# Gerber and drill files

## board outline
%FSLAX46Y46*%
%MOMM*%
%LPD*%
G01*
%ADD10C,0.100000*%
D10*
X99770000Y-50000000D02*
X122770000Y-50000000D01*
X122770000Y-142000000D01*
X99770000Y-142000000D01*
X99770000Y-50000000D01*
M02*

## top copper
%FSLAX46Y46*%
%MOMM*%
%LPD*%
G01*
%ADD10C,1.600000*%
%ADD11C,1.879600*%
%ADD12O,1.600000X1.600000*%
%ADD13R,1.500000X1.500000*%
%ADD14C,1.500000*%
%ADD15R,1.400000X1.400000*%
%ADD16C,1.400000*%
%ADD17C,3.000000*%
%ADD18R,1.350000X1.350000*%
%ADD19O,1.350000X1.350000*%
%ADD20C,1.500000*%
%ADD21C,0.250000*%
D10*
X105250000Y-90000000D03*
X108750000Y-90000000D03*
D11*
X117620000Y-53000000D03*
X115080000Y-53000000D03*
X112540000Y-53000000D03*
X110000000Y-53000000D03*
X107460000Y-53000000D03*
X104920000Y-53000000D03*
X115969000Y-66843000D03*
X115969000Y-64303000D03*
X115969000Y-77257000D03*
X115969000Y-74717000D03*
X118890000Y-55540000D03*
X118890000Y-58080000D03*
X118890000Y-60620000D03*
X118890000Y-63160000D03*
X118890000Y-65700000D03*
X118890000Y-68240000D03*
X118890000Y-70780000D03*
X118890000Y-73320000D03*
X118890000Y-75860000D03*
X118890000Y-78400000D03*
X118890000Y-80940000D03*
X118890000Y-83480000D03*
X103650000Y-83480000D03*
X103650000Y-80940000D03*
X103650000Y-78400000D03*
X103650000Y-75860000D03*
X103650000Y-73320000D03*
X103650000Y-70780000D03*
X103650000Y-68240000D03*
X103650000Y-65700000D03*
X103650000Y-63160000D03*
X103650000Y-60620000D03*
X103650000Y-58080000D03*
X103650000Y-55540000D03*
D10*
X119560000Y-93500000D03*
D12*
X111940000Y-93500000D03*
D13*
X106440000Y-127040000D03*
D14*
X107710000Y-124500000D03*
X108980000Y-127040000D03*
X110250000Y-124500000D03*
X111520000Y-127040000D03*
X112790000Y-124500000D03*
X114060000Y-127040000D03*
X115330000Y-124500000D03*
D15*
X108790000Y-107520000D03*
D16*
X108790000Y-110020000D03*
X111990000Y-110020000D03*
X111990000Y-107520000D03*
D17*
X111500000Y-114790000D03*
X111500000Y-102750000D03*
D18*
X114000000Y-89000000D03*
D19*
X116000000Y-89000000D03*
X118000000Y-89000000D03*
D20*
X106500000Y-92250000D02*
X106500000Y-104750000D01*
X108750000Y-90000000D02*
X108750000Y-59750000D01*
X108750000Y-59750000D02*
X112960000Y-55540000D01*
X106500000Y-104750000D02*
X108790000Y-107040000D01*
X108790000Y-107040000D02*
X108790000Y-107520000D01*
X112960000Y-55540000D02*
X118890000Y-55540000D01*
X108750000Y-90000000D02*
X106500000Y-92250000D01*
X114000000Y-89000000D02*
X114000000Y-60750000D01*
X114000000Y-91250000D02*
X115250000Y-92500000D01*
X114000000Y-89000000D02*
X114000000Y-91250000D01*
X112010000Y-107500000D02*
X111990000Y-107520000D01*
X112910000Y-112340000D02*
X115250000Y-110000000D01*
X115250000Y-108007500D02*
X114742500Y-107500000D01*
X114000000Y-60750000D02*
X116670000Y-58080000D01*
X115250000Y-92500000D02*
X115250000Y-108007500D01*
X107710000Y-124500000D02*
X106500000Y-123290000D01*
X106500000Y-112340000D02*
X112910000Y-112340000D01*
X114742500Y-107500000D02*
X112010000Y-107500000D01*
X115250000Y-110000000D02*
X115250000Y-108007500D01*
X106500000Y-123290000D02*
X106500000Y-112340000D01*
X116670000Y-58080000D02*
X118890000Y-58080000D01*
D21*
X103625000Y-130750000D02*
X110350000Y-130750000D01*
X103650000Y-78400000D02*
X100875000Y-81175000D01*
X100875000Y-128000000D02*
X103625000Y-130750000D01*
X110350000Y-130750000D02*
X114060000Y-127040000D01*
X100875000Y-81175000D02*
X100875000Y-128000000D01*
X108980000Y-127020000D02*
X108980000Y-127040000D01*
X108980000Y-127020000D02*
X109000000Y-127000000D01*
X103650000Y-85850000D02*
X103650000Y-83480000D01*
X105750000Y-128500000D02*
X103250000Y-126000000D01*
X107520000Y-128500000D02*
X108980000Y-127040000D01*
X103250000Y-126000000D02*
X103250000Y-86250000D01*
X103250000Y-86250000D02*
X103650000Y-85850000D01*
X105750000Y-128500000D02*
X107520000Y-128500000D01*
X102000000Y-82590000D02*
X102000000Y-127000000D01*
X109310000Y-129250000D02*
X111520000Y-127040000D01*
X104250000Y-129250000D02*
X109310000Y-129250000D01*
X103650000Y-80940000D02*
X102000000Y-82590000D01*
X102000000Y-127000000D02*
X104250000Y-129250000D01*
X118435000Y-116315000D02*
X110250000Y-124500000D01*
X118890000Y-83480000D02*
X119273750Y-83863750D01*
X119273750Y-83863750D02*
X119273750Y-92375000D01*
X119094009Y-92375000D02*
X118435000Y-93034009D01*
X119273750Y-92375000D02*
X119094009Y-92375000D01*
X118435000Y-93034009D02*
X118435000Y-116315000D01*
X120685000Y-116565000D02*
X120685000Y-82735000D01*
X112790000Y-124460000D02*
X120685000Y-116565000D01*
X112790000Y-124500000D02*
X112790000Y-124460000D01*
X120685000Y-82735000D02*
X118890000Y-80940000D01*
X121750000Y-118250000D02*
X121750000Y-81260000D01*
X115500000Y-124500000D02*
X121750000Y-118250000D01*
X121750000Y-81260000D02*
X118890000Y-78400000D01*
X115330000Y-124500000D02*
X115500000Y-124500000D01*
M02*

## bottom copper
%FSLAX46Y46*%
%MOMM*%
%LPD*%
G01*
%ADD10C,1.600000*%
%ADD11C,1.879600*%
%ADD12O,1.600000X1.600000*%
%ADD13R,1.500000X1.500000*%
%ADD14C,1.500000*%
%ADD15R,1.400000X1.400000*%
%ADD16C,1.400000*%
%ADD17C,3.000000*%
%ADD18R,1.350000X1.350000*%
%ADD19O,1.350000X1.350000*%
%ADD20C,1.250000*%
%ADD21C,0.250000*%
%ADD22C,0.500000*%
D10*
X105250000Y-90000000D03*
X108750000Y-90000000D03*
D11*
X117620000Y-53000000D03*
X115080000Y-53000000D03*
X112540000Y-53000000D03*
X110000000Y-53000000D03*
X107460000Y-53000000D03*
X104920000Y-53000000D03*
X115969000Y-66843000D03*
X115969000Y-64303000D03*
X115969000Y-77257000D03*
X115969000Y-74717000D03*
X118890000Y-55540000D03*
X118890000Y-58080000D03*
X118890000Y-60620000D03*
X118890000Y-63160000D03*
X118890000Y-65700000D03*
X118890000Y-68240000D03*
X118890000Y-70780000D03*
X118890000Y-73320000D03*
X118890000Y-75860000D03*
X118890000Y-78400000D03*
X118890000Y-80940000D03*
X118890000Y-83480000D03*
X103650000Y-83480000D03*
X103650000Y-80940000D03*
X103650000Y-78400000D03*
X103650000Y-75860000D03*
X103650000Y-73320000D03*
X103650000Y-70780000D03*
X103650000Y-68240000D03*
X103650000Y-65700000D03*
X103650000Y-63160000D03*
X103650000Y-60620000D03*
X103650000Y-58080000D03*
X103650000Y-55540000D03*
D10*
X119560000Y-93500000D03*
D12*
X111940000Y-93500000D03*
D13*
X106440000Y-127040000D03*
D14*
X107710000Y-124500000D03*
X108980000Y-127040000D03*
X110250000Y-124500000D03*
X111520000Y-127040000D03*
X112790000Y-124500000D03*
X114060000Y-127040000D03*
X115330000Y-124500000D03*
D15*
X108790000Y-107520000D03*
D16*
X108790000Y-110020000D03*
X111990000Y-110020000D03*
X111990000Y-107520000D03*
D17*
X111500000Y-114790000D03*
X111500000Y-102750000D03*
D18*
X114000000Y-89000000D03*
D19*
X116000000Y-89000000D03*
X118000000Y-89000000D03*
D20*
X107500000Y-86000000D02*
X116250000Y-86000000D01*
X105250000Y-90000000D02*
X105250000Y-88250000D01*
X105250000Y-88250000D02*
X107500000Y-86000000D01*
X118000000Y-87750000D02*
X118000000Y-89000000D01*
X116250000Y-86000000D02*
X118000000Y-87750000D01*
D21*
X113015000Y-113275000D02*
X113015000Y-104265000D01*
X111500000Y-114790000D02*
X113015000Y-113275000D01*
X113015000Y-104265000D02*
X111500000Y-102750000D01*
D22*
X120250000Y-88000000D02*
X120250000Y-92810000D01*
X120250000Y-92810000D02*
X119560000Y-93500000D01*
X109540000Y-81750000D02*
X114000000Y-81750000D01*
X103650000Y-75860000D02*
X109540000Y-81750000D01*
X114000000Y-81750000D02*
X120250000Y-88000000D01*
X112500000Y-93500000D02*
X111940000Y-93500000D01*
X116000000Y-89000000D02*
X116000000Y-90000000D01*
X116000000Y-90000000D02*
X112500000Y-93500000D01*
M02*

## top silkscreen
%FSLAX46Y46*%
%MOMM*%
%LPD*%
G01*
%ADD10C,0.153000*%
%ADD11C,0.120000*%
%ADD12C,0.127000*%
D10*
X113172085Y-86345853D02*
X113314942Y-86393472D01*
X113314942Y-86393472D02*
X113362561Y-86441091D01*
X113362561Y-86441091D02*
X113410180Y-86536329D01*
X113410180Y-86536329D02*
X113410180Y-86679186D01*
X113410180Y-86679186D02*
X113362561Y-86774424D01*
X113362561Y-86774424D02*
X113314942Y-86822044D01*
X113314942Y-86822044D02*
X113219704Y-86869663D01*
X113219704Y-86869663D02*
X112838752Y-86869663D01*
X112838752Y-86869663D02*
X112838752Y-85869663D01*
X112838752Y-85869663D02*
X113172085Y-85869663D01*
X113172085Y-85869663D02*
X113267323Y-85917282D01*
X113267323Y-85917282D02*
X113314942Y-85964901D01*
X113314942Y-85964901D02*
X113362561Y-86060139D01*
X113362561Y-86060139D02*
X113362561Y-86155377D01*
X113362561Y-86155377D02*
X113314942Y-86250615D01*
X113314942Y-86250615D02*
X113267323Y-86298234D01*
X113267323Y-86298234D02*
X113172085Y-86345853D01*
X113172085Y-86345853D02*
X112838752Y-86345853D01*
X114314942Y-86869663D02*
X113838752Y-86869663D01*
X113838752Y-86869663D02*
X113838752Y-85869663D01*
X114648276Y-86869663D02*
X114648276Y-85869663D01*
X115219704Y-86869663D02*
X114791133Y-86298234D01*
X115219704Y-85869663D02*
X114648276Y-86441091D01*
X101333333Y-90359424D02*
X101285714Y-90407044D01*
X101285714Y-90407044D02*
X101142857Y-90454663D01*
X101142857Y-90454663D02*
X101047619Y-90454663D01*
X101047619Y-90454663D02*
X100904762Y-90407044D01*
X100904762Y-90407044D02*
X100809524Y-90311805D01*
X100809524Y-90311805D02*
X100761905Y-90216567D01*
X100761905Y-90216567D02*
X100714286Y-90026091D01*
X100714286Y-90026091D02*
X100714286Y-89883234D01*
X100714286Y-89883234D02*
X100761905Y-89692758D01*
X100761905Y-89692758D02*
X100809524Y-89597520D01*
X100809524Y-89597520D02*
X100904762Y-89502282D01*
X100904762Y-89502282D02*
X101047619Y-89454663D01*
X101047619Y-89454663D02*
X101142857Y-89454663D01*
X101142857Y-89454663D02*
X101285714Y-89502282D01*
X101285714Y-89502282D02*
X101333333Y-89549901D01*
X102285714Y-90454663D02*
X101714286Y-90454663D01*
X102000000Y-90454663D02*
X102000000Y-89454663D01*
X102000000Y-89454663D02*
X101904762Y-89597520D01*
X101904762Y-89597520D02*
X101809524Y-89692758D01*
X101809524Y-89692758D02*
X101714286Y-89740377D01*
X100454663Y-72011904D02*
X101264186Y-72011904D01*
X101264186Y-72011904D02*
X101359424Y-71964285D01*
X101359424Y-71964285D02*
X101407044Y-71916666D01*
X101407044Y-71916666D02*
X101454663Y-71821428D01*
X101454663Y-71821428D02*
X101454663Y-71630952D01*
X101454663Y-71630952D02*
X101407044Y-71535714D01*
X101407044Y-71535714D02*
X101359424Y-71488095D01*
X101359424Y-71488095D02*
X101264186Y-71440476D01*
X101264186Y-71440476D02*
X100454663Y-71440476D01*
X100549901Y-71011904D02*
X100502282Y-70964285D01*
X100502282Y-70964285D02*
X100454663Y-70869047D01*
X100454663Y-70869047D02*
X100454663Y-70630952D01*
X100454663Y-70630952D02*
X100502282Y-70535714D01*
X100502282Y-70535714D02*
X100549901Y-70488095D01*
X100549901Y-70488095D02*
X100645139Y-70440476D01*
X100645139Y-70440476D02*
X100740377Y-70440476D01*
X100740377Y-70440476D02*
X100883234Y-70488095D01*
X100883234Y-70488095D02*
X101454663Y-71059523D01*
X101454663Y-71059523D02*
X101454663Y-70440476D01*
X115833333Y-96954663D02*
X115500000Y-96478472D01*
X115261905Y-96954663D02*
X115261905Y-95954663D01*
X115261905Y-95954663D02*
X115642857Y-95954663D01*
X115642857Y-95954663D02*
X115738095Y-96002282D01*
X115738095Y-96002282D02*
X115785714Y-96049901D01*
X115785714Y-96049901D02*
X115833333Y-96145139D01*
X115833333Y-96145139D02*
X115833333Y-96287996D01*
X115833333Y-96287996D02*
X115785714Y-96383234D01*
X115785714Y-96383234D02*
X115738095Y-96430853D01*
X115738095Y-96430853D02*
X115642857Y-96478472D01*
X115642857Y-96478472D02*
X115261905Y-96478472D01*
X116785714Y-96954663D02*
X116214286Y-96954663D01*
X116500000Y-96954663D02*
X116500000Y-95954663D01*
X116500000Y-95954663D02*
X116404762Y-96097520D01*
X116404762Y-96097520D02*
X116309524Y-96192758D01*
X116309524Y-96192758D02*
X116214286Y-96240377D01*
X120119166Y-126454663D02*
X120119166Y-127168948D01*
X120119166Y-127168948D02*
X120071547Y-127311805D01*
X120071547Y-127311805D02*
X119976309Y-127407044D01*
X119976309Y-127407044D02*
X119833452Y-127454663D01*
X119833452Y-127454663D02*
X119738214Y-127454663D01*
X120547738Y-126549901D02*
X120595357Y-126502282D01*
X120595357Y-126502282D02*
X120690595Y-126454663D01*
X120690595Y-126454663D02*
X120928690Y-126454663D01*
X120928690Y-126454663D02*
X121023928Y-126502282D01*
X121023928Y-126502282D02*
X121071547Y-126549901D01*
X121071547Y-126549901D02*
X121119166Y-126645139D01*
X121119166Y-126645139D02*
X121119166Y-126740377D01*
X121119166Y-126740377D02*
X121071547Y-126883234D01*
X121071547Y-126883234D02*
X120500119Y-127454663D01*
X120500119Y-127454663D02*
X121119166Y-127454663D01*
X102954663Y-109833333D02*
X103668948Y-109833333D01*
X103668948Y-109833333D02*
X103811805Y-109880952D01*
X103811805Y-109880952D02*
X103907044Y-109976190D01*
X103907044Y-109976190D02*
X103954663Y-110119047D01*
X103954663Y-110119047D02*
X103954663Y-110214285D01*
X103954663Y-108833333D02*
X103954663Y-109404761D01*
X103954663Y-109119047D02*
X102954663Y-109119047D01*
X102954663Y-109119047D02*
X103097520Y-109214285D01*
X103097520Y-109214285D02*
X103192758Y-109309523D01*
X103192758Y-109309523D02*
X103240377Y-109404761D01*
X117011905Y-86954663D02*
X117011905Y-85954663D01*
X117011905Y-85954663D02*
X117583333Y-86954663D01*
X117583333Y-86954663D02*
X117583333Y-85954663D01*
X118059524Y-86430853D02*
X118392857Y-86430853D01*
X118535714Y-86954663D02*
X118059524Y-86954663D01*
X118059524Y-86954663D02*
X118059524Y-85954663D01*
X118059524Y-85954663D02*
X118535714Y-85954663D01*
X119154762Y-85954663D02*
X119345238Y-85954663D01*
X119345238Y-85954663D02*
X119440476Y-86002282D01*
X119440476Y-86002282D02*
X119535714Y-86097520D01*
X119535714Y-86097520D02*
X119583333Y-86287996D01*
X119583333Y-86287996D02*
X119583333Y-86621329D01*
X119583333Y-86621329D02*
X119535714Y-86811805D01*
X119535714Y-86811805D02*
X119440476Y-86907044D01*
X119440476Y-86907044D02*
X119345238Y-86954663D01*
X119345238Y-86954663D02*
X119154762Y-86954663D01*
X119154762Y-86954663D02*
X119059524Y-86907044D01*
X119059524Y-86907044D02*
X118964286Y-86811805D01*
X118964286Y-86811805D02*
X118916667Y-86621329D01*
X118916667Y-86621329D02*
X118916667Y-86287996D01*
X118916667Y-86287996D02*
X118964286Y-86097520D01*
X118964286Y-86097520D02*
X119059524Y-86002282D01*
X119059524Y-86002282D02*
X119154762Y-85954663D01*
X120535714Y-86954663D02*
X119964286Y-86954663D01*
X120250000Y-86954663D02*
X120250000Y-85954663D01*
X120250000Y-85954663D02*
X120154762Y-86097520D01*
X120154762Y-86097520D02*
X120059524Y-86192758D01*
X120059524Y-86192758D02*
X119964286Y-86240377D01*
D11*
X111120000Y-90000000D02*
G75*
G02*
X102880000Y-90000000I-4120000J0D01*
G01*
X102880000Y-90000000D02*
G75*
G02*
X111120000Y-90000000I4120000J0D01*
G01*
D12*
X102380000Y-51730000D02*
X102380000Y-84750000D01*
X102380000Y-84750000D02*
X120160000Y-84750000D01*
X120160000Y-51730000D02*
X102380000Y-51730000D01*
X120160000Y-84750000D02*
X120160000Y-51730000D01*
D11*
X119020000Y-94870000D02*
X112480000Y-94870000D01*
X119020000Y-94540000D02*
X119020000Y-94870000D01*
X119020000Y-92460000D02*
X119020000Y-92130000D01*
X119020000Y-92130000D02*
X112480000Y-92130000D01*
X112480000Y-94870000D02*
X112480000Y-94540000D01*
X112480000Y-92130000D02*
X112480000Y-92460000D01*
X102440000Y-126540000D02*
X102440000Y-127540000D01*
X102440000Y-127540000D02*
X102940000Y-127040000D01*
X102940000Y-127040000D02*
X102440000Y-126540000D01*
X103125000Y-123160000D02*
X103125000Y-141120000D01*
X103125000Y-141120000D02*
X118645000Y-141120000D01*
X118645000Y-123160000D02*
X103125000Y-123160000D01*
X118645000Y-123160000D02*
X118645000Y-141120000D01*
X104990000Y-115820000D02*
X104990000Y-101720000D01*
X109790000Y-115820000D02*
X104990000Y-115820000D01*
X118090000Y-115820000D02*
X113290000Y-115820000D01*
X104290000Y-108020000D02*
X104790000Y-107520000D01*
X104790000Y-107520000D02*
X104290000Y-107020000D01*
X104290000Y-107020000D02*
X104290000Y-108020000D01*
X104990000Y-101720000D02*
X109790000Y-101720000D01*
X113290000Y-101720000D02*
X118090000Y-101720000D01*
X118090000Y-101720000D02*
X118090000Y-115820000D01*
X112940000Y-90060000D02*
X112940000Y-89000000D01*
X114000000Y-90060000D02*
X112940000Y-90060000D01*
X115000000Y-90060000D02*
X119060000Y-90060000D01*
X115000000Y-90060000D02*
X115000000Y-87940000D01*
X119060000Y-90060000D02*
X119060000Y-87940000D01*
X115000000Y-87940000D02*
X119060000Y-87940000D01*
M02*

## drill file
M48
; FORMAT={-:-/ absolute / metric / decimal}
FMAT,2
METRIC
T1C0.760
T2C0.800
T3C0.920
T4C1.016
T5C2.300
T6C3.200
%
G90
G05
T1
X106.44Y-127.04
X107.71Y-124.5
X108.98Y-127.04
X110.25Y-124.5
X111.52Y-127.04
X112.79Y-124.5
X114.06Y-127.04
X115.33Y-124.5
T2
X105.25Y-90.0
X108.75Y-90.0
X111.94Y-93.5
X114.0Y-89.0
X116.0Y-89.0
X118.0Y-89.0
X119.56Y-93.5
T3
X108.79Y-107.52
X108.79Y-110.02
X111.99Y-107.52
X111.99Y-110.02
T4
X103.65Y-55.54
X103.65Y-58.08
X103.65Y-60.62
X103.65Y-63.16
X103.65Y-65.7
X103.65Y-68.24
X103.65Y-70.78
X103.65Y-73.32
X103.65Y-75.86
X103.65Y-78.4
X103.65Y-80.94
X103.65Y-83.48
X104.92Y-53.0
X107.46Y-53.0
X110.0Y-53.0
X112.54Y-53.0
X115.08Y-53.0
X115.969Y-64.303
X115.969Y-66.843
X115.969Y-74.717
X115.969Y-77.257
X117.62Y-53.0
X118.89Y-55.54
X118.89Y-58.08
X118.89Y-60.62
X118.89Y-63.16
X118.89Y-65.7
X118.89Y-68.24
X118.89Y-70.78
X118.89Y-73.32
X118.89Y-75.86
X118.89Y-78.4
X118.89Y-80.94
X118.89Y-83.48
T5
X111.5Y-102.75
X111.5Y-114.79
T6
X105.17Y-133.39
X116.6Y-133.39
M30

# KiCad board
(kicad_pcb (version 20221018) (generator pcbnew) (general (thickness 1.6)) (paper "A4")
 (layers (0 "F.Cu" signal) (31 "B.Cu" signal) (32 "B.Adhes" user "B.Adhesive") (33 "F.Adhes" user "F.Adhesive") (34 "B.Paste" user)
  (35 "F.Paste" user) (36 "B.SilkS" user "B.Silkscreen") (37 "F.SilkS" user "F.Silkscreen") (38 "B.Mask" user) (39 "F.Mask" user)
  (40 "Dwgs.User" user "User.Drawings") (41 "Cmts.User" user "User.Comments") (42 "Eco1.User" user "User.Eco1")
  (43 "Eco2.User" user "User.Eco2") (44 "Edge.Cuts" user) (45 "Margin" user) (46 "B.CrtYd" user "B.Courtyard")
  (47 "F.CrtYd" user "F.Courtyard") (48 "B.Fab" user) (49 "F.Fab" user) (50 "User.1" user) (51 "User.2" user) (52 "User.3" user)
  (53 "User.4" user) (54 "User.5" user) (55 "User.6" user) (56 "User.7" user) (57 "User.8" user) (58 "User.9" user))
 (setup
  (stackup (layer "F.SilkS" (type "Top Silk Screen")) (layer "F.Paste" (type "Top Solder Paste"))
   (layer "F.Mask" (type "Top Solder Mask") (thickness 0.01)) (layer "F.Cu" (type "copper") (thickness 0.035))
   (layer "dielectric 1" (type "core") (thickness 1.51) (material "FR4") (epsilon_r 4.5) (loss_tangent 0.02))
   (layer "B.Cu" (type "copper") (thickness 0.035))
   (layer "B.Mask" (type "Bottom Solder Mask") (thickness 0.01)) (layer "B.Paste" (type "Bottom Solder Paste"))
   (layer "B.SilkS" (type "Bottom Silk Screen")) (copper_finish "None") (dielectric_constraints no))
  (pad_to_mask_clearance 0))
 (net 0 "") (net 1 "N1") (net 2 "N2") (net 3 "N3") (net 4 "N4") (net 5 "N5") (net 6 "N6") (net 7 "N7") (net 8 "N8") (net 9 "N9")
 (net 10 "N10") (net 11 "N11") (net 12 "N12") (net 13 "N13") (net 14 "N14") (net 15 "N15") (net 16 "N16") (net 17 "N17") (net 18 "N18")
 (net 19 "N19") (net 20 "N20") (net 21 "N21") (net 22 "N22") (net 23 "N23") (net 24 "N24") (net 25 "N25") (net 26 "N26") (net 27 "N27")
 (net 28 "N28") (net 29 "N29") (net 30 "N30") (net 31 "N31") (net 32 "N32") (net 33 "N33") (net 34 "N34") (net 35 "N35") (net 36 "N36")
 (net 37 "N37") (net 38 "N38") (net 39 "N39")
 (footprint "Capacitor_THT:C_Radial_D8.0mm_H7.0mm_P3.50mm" (layer "F.Cu") (at 105.25 90)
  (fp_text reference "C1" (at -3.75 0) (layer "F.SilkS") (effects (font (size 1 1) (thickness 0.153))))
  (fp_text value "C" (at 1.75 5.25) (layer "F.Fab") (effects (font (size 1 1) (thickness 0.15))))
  (fp_circle (center 1.75 0) (end 5.87 0) (stroke (width 0.12) (type solid)) (fill none) (layer "F.SilkS"))
  (pad "1" thru_hole circle (at 0 0) (size 1.6 1.6) (drill 0.8) (layers "*.Cu" "*.Mask") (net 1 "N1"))
  (pad "2" thru_hole circle (at 3.5 0) (size 1.6 1.6) (drill 0.8) (layers "*.Cu" "*.Mask") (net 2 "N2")))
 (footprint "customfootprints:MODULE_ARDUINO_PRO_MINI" (layer "F.Cu") (at 111.27 68.24)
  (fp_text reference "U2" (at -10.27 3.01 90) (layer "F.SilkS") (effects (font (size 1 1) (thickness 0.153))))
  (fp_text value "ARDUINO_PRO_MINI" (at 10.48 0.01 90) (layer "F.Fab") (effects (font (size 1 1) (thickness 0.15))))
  (fp_line (start -8.89 -16.51) (end -8.89 16.51) (stroke (width 0.127) (type solid)) (layer "F.SilkS"))
  (fp_line (start -8.89 16.51) (end 8.89 16.51) (stroke (width 0.127) (type solid)) (layer "F.SilkS"))
  (fp_line (start 8.89 -16.51) (end -8.89 -16.51) (stroke (width 0.127) (type solid)) (layer "F.SilkS"))
  (fp_line (start 8.89 16.51) (end 8.89 -16.51) (stroke (width 0.127) (type solid)) (layer "F.SilkS"))
  (pad "JP1_1" thru_hole circle (at 6.35 -15.24) (size 1.8796 1.8796) (drill 1.016) (layers "*.Cu" "*.Mask") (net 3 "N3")
   (solder_mask_margin 0.102))
  (pad "JP1_2" thru_hole circle (at 3.81 -15.24) (size 1.8796 1.8796) (drill 1.016) (layers "*.Cu" "*.Mask") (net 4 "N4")
   (solder_mask_margin 0.102))
  (pad "JP1_3" thru_hole circle (at 1.27 -15.24) (size 1.8796 1.8796) (drill 1.016) (layers "*.Cu" "*.Mask") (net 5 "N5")
   (solder_mask_margin 0.102))
  (pad "JP1_4" thru_hole circle (at -1.27 -15.24) (size 1.8796 1.8796) (drill 1.016) (layers "*.Cu" "*.Mask") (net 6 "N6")
   (solder_mask_margin 0.102))
  (pad "JP1_5" thru_hole circle (at -3.81 -15.24) (size 1.8796 1.8796) (drill 1.016) (layers "*.Cu" "*.Mask") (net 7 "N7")
   (solder_mask_margin 0.102))
  (pad "JP1_6" thru_hole circle (at -6.35 -15.24) (size 1.8796 1.8796) (drill 1.016) (layers "*.Cu" "*.Mask") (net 7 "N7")
   (solder_mask_margin 0.102))
  (pad "JP2_1" thru_hole circle (at 4.699 -1.397) (size 1.8796 1.8796) (drill 1.016) (layers "*.Cu" "*.Mask") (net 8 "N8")
   (solder_mask_margin 0.102))
  (pad "JP2_2" thru_hole circle (at 4.699 -3.937) (size 1.8796 1.8796) (drill 1.016) (layers "*.Cu" "*.Mask") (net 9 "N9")
   (solder_mask_margin 0.102))
  (pad "JP3_1" thru_hole circle (at 4.699 9.017) (size 1.8796 1.8796) (drill 1.016) (layers "*.Cu" "*.Mask") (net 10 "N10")
   (solder_mask_margin 0.102))
  (pad "JP3_2" thru_hole circle (at 4.699 6.477) (size 1.8796 1.8796) (drill 1.016) (layers "*.Cu" "*.Mask") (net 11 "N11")
   (solder_mask_margin 0.102))
  (pad "JP6_1" thru_hole circle (at 7.62 -12.7) (size 1.8796 1.8796) (drill 1.016) (layers "*.Cu" "*.Mask") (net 2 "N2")
   (solder_mask_margin 0.102))
  (pad "JP6_2" thru_hole circle (at 7.62 -10.16) (size 1.8796 1.8796) (drill 1.016) (layers "*.Cu" "*.Mask") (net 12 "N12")
   (solder_mask_margin 0.102))
  (pad "JP6_3" thru_hole circle (at 7.62 -7.62) (size 1.8796 1.8796) (drill 1.016) (layers "*.Cu" "*.Mask") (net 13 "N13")
   (solder_mask_margin 0.102))
  (pad "JP6_4" thru_hole circle (at 7.62 -5.08) (size 1.8796 1.8796) (drill 1.016) (layers "*.Cu" "*.Mask") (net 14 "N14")
   (solder_mask_margin 0.102))
  (pad "JP6_5" thru_hole circle (at 7.62 -2.54) (size 1.8796 1.8796) (drill 1.016) (layers "*.Cu" "*.Mask") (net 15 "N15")
   (solder_mask_margin 0.102))
  (pad "JP6_6" thru_hole circle (at 7.62 0) (size 1.8796 1.8796) (drill 1.016) (layers "*.Cu" "*.Mask") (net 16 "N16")
   (solder_mask_margin 0.102))
  (pad "JP6_7" thru_hole circle (at 7.62 2.54) (size 1.8796 1.8796) (drill 1.016) (layers "*.Cu" "*.Mask") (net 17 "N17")
   (solder_mask_margin 0.102))
  (pad "JP6_8" thru_hole circle (at 7.62 5.08) (size 1.8796 1.8796) (drill 1.016) (layers "*.Cu" "*.Mask") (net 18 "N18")
   (solder_mask_margin 0.102))
  (pad "JP6_9" thru_hole circle (at 7.62 7.62) (size 1.8796 1.8796) (drill 1.016) (layers "*.Cu" "*.Mask") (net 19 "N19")
   (solder_mask_margin 0.102))
  (pad "JP6_10" thru_hole circle (at 7.62 10.16) (size 1.8796 1.8796) (drill 1.016) (layers "*.Cu" "*.Mask") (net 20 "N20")
   (solder_mask_margin 0.102))
  (pad "JP6_11" thru_hole circle (at 7.62 12.7) (size 1.8796 1.8796) (drill 1.016) (layers "*.Cu" "*.Mask") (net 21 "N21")
   (solder_mask_margin 0.102))
  (pad "JP6_12" thru_hole circle (at 7.62 15.24) (size 1.8796 1.8796) (drill 1.016) (layers "*.Cu" "*.Mask") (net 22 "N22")
   (solder_mask_margin 0.102))
  (pad "JP7_1" thru_hole circle (at -7.62 15.24) (size 1.8796 1.8796) (drill 1.016) (layers "*.Cu" "*.Mask") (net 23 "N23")
   (solder_mask_margin 0.102))
  (pad "JP7_2" thru_hole circle (at -7.62 12.7) (size 1.8796 1.8796) (drill 1.016) (layers "*.Cu" "*.Mask") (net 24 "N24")
   (solder_mask_margin 0.102))
  (pad "JP7_3" thru_hole circle (at -7.62 10.16) (size 1.8796 1.8796) (drill 1.016) (layers "*.Cu" "*.Mask") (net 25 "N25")
   (solder_mask_margin 0.102))
  (pad "JP7_4" thru_hole circle (at -7.62 7.62) (size 1.8796 1.8796) (drill 1.016) (layers "*.Cu" "*.Mask") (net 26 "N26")
   (solder_mask_margin 0.102))
  (pad "JP7_5" thru_hole circle (at -7.62 5.08) (size 1.8796 1.8796) (drill 1.016) (layers "*.Cu" "*.Mask") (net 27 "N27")
   (solder_mask_margin 0.102))
  (pad "JP7_6" thru_hole circle (at -7.62 2.54) (size 1.8796 1.8796) (drill 1.016) (layers "*.Cu" "*.Mask") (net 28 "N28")
   (solder_mask_margin 0.102))
  (pad "JP7_7" thru_hole circle (at -7.62 0) (size 1.8796 1.8796) (drill 1.016) (layers "*.Cu" "*.Mask") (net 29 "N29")
   (solder_mask_margin 0.102))
  (pad "JP7_8" thru_hole circle (at -7.62 -2.54) (size 1.8796 1.8796) (drill 1.016) (layers "*.Cu" "*.Mask") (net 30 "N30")
   (solder_mask_margin 0.102))
  (pad "JP7_9" thru_hole circle (at -7.62 -5.08) (size 1.8796 1.8796) (drill 1.016) (layers "*.Cu" "*.Mask") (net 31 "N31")
   (solder_mask_margin 0.102))
  (pad "JP7_10" thru_hole circle (at -7.62 -7.62) (size 1.8796 1.8796) (drill 1.016) (layers "*.Cu" "*.Mask") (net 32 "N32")
   (solder_mask_margin 0.102))
  (pad "JP7_11" thru_hole circle (at -7.62 -10.16) (size 1.8796 1.8796) (drill 1.016) (layers "*.Cu" "*.Mask") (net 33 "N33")
   (solder_mask_margin 0.102))
  (pad "JP7_12" thru_hole circle (at -7.62 -12.7) (size 1.8796 1.8796) (drill 1.016) (layers "*.Cu" "*.Mask") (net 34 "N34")
   (solder_mask_margin 0.102)))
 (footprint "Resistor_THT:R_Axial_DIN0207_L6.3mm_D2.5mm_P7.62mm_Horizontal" (layer "F.Cu") (at 119.56 93.5 180)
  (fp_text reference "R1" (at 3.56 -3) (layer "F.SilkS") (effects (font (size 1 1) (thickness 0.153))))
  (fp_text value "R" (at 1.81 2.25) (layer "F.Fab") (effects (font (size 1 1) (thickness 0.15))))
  (fp_line (start 0.54 -1.37) (end 7.08 -1.37) (stroke (width 0.12) (type solid)) (layer "F.SilkS"))
  (fp_line (start 0.54 -1.04) (end 0.54 -1.37) (stroke (width 0.12) (type solid)) (layer "F.SilkS"))
  (fp_line (start 0.54 1.04) (end 0.54 1.37) (stroke (width 0.12) (type solid)) (layer "F.SilkS"))
  (fp_line (start 0.54 1.37) (end 7.08 1.37) (stroke (width 0.12) (type solid)) (layer "F.SilkS"))
  (fp_line (start 7.08 -1.37) (end 7.08 -1.04) (stroke (width 0.12) (type solid)) (layer "F.SilkS"))
  (fp_line (start 7.08 1.37) (end 7.08 1.04) (stroke (width 0.12) (type solid)) (layer "F.SilkS"))
  (pad "1" thru_hole circle (at 0 0 180) (size 1.6 1.6) (drill 0.8) (layers "*.Cu" "*.Mask") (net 26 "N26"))
  (pad "2" thru_hole oval (at 7.62 0 180) (size 1.6 1.6) (drill 0.8) (layers "*.Cu" "*.Mask") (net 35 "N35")))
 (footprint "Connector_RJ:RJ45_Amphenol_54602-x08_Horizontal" (layer "F.Cu") (at 106.44 127.04)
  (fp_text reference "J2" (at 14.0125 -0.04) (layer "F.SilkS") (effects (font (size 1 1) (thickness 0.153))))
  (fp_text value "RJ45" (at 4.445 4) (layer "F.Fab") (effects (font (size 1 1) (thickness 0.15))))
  (fp_line (start -4 -0.5) (end -4 0.5) (stroke (width 0.12) (type solid)) (layer "F.SilkS"))
  (fp_line (start -4 0.5) (end -3.5 0) (stroke (width 0.12) (type solid)) (layer "F.SilkS"))
  (fp_line (start -3.5 0) (end -4 -0.5) (stroke (width 0.12) (type solid)) (layer "F.SilkS"))
  (fp_line (start -3.315 -3.88) (end -3.315 14.08) (stroke (width 0.12) (type solid)) (layer "F.SilkS"))
  (fp_line (start -3.315 14.08) (end 12.205 14.08) (stroke (width 0.12) (type solid)) (layer "F.SilkS"))
  (fp_line (start 12.205 -3.88) (end -3.315 -3.88) (stroke (width 0.12) (type solid)) (layer "F.SilkS"))
  (fp_line (start 12.205 -3.88) (end 12.205 14.08) (stroke (width 0.12) (type solid)) (layer "F.SilkS"))
  (pad "" np_thru_hole circle (at -1.27 6.35) (size 3.2 3.2) (drill 3.2) (layers "*.Cu" "*.Mask"))
  (pad "" np_thru_hole circle (at 10.16 6.35) (size 3.2 3.2) (drill 3.2) (layers "*.Cu" "*.Mask"))
  (pad "1" thru_hole rect (at 0 0) (size 1.5 1.5) (drill 0.76) (layers "*.Cu" "*.Mask") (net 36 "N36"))
  (pad "2" thru_hole circle (at 1.27 -2.54) (size 1.5 1.5) (drill 0.76) (layers "*.Cu" "*.Mask") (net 12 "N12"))
  (pad "3" thru_hole circle (at 2.54 0) (size 1.5 1.5) (drill 0.76) (layers "*.Cu" "*.Mask") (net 23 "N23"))
  (pad "4" thru_hole circle (at 3.81 -2.54) (size 1.5 1.5) (drill 0.76) (layers "*.Cu" "*.Mask") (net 22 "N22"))
  (pad "5" thru_hole circle (at 5.08 0) (size 1.5 1.5) (drill 0.76) (layers "*.Cu" "*.Mask") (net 24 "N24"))
  (pad "6" thru_hole circle (at 6.35 -2.54) (size 1.5 1.5) (drill 0.76) (layers "*.Cu" "*.Mask") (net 21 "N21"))
  (pad "7" thru_hole circle (at 7.62 0) (size 1.5 1.5) (drill 0.76) (layers "*.Cu" "*.Mask") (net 25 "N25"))
  (pad "8" thru_hole circle (at 8.89 -2.54) (size 1.5 1.5) (drill 0.76) (layers "*.Cu" "*.Mask") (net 20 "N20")))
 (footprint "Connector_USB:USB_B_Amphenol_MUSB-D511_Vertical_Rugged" (layer "F.Cu") (at 108.79 107.52 90)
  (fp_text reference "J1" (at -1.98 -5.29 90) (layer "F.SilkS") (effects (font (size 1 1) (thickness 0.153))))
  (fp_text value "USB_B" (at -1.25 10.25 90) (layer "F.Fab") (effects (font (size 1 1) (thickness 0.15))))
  (fp_line (start -8.3 -3.8) (end 5.8 -3.8) (stroke (width 0.12) (type solid)) (layer "F.SilkS"))
  (fp_line (start -8.3 1) (end -8.3 -3.8) (stroke (width 0.12) (type solid)) (layer "F.SilkS"))
  (fp_line (start -8.3 9.3) (end -8.3 4.5) (stroke (width 0.12) (type solid)) (layer "F.SilkS"))
  (fp_line (start -0.5 -4.5) (end 0 -4) (stroke (width 0.12) (type solid)) (layer "F.SilkS"))
  (fp_line (start 0 -4) (end 0.5 -4.5) (stroke (width 0.12) (type solid)) (layer "F.SilkS"))
  (fp_line (start 0.5 -4.5) (end -0.5 -4.5) (stroke (width 0.12) (type solid)) (layer "F.SilkS"))
  (fp_line (start 5.8 -3.8) (end 5.8 1) (stroke (width 0.12) (type solid)) (layer "F.SilkS"))
  (fp_line (start 5.8 4.5) (end 5.8 9.3) (stroke (width 0.12) (type solid)) (layer "F.SilkS"))
  (fp_line (start 5.8 9.3) (end -8.3 9.3) (stroke (width 0.12) (type solid)) (layer "F.SilkS"))
  (pad "1" thru_hole rect (at 0 0 90) (size 1.4 1.4) (drill 0.92) (layers "*.Cu" "*.Mask") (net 2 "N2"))
  (pad "2" thru_hole circle (at -2.5 0 90) (size 1.4 1.4) (drill 0.92) (layers "*.Cu" "*.Mask") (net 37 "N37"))
  (pad "3" thru_hole circle (at -2.5 3.2 90) (size 1.4 1.4) (drill 0.92) (layers "*.Cu" "*.Mask") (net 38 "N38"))
  (pad "4" thru_hole circle (at 0 3.2 90) (size 1.4 1.4) (drill 0.92) (layers "*.Cu" "*.Mask") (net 12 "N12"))
  (pad "5" thru_hole circle (at -7.27 2.71 90) (size 3 3) (drill 2.3) (layers "*.Cu" "*.Mask") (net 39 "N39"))
  (pad "5" thru_hole circle (at 4.77 2.71 90) (size 3 3) (drill 2.3) (layers "*.Cu" "*.Mask") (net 39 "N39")))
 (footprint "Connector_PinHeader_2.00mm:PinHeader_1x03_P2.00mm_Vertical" (layer "F.Cu") (at 114 89 90)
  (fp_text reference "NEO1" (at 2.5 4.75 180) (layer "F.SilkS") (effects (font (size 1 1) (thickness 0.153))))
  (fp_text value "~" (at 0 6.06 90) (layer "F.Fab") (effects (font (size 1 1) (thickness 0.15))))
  (fp_line (start -1.06 -1.06) (end 0 -1.06) (stroke (width 0.12) (type solid)) (layer "F.SilkS"))
  (fp_line (start -1.06 0) (end -1.06 -1.06) (stroke (width 0.12) (type solid)) (layer "F.SilkS"))
  (fp_line (start -1.06 1) (end -1.06 5.06) (stroke (width 0.12) (type solid)) (layer "F.SilkS"))
  (fp_line (start -1.06 1) (end 1.06 1) (stroke (width 0.12) (type solid)) (layer "F.SilkS"))
  (fp_line (start -1.06 5.06) (end 1.06 5.06) (stroke (width 0.12) (type solid)) (layer "F.SilkS"))
  (fp_line (start 1.06 1) (end 1.06 5.06) (stroke (width 0.12) (type solid)) (layer "F.SilkS"))
  (pad "1" thru_hole rect (at 0 0 90) (size 1.35 1.35) (drill 0.8) (layers "*.Cu" "*.Mask") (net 12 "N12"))
  (pad "2" thru_hole oval (at 0 2 90) (size 1.35 1.35) (drill 0.8) (layers "*.Cu" "*.Mask") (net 35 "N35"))
  (pad "3" thru_hole oval (at 0 4 90) (size 1.35 1.35) (drill 0.8) (layers "*.Cu" "*.Mask") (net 1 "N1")))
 (gr_rect (start 99.77 50) (end 122.77 142) (stroke (width 0.1) (type default)) (fill none) (layer "Edge.Cuts"))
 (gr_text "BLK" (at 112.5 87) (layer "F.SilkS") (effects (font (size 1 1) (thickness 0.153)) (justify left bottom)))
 (segment (start 107.5 86) (end 116.25 86) (width 1.25) (layer "B.Cu") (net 1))
 (segment (start 105.25 90) (end 105.25 88.25) (width 1.25) (layer "B.Cu") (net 1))
 (segment (start 105.25 88.25) (end 107.5 86) (width 1.25) (layer "B.Cu") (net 1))
 (segment (start 118 87.75) (end 118 89) (width 1.25) (layer "B.Cu") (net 1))
 (segment (start 116.25 86) (end 118 87.75) (width 1.25) (layer "B.Cu") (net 1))
 (segment (start 106.5 92.25) (end 106.5 104.75) (width 1.5) (layer "F.Cu") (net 2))
 (segment (start 108.75 90) (end 108.75 59.75) (width 1.5) (layer "F.Cu") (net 2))
 (segment (start 108.75 59.75) (end 112.96 55.54) (width 1.5) (layer "F.Cu") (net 2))
 (segment (start 106.5 104.75) (end 108.79 107.04) (width 1.5) (layer "F.Cu") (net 2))
 (segment (start 108.79 107.04) (end 108.79 107.52) (width 1.5) (layer "F.Cu") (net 2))
 (segment (start 112.96 55.54) (end 118.89 55.54) (width 1.5) (layer "F.Cu") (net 2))
 (segment (start 108.75 90) (end 106.5 92.25) (width 1.5) (layer "F.Cu") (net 2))
 (segment (start 114 89) (end 114 60.75) (width 1.5) (layer "F.Cu") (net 12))
 (segment (start 114 91.25) (end 115.25 92.5) (width 1.5) (layer "F.Cu") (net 12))
 (segment (start 114 89) (end 114 91.25) (width 1.5) (layer "F.Cu") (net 12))
 (segment (start 112.01 107.5) (end 111.99 107.52) (width 1.5) (layer "F.Cu") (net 12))
 (segment (start 112.91 112.34) (end 115.25 110) (width 1.5) (layer "F.Cu") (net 12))
 (segment (start 115.25 108.0075) (end 114.7425 107.5) (width 1.5) (layer "F.Cu") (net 12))
 (segment (start 114 60.75) (end 116.67 58.08) (width 1.5) (layer "F.Cu") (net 12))
 (segment (start 115.25 92.5) (end 115.25 108.0075) (width 1.5) (layer "F.Cu") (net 12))
 (segment (start 107.71 124.5) (end 106.5 123.29) (width 1.5) (layer "F.Cu") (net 12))
 (segment (start 106.5 112.34) (end 112.91 112.34) (width 1.5) (layer "F.Cu") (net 12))
 (segment (start 114.7425 107.5) (end 112.01 107.5) (width 1.5) (layer "F.Cu") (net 12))
 (segment (start 115.25 110) (end 115.25 108.0075) (width 1.5) (layer "F.Cu") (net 12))
 (segment (start 106.5 123.29) (end 106.5 112.34) (width 1.5) (layer "F.Cu") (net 12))
 (segment (start 116.67 58.08) (end 118.89 58.08) (width 1.5) (layer "F.Cu") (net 12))
 (segment (start 113.015 113.275) (end 113.015 104.265) (width 0.25) (layer "B.Cu") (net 39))
 (segment (start 111.5 114.79) (end 113.015 113.275) (width 0.25) (layer "B.Cu") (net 39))
 (segment (start 113.015 104.265) (end 111.5 102.75) (width 0.25) (layer "B.Cu") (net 39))
 (segment (start 103.625 130.75) (end 110.35 130.75) (width 0.25) (layer "F.Cu") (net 25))
 (segment (start 103.65 78.4) (end 100.875 81.175) (width 0.25) (layer "F.Cu") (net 25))
 (segment (start 100.875 128) (end 103.625 130.75) (width 0.25) (layer "F.Cu") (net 25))
 (segment (start 110.35 130.75) (end 114.06 127.04) (width 0.25) (layer "F.Cu") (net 25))
 (segment (start 100.875 81.175) (end 100.875 128) (width 0.25) (layer "F.Cu") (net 25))
 (segment (start 120.25 88) (end 120.25 92.81) (width 0.5) (layer "B.Cu") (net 26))
 (segment (start 120.25 92.81) (end 119.56 93.5) (width 0.5) (layer "B.Cu") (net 26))
 (segment (start 109.54 81.75) (end 114 81.75) (width 0.5) (layer "B.Cu") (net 26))
 (segment (start 103.65 75.86) (end 109.54 81.75) (width 0.5) (layer "B.Cu") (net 26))
 (segment (start 114 81.75) (end 120.25 88) (width 0.5) (layer "B.Cu") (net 26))
 (segment (start 112.5 93.5) (end 111.94 93.5) (width 0.5) (layer "B.Cu") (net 35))
 (segment (start 116 89) (end 116 90) (width 0.5) (layer "B.Cu") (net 35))
 (segment (start 116 90) (end 112.5 93.5) (width 0.5) (layer "B.Cu") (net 35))
 (segment (start 108.98 127.02) (end 108.98 127.04) (width 0.25) (layer "F.Cu") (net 23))
 (segment (start 108.98 127.02) (end 109 127) (width 0.25) (layer "F.Cu") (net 23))
 (segment (start 103.65 85.85) (end 103.65 83.48) (width 0.25) (layer "F.Cu") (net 23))
 (segment (start 105.75 128.5) (end 103.25 126) (width 0.25) (layer "F.Cu") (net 23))
 (segment (start 107.52 128.5) (end 108.98 127.04) (width 0.25) (layer "F.Cu") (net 23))
 (segment (start 103.25 126) (end 103.25 86.25) (width 0.25) (layer "F.Cu") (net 23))
 (segment (start 103.25 86.25) (end 103.65 85.85) (width 0.25) (layer "F.Cu") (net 23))
 (segment (start 105.75 128.5) (end 107.52 128.5) (width 0.25) (layer "F.Cu") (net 23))
 (segment (start 102 82.59) (end 102 127) (width 0.25) (layer "F.Cu") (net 24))
 (segment (start 109.31 129.25) (end 111.52 127.04) (width 0.25) (layer "F.Cu") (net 24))
 (segment (start 104.25 129.25) (end 109.31 129.25) (width 0.25) (layer "F.Cu") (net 24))
 (segment (start 103.65 80.94) (end 102 82.59) (width 0.25) (layer "F.Cu") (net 24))
 (segment (start 102 127) (end 104.25 129.25) (width 0.25) (layer "F.Cu") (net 24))
 (segment (start 118.435 116.315) (end 110.25 124.5) (width 0.25) (layer "F.Cu") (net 22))
 (segment (start 118.89 83.48) (end 119.27375 83.86375) (width 0.25) (layer "F.Cu") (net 22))
 (segment (start 119.27375 83.86375) (end 119.27375 92.375) (width 0.25) (layer "F.Cu") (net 22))
 (segment (start 119.094009 92.375) (end 118.435 93.034009) (width 0.25) (layer "F.Cu") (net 22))
 (segment (start 119.27375 92.375) (end 119.094009 92.375) (width 0.25) (layer "F.Cu") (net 22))
 (segment (start 118.435 93.034009) (end 118.435 116.315) (width 0.25) (layer "F.Cu") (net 22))
 (segment (start 120.685 116.565) (end 120.685 82.735) (width 0.25) (layer "F.Cu") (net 21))
 (segment (start 112.79 124.46) (end 120.685 116.565) (width 0.25) (layer "F.Cu") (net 21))
 (segment (start 112.79 124.5) (end 112.79 124.46) (width 0.25) (layer "F.Cu") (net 21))
 (segment (start 120.685 82.735) (end 118.89 80.94) (width 0.25) (layer "F.Cu") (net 21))
 (segment (start 121.75 118.25) (end 121.75 81.26) (width 0.25) (layer "F.Cu") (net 20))
 (segment (start 115.5 124.5) (end 121.75 118.25) (width 0.25) (layer "F.Cu") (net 20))
 (segment (start 121.75 81.26) (end 118.89 78.4) (width 0.25) (layer "F.Cu") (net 20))
 (segment (start 115.33 124.5) (end 115.5 124.5) (width 0.25) (layer "F.Cu") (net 20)))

